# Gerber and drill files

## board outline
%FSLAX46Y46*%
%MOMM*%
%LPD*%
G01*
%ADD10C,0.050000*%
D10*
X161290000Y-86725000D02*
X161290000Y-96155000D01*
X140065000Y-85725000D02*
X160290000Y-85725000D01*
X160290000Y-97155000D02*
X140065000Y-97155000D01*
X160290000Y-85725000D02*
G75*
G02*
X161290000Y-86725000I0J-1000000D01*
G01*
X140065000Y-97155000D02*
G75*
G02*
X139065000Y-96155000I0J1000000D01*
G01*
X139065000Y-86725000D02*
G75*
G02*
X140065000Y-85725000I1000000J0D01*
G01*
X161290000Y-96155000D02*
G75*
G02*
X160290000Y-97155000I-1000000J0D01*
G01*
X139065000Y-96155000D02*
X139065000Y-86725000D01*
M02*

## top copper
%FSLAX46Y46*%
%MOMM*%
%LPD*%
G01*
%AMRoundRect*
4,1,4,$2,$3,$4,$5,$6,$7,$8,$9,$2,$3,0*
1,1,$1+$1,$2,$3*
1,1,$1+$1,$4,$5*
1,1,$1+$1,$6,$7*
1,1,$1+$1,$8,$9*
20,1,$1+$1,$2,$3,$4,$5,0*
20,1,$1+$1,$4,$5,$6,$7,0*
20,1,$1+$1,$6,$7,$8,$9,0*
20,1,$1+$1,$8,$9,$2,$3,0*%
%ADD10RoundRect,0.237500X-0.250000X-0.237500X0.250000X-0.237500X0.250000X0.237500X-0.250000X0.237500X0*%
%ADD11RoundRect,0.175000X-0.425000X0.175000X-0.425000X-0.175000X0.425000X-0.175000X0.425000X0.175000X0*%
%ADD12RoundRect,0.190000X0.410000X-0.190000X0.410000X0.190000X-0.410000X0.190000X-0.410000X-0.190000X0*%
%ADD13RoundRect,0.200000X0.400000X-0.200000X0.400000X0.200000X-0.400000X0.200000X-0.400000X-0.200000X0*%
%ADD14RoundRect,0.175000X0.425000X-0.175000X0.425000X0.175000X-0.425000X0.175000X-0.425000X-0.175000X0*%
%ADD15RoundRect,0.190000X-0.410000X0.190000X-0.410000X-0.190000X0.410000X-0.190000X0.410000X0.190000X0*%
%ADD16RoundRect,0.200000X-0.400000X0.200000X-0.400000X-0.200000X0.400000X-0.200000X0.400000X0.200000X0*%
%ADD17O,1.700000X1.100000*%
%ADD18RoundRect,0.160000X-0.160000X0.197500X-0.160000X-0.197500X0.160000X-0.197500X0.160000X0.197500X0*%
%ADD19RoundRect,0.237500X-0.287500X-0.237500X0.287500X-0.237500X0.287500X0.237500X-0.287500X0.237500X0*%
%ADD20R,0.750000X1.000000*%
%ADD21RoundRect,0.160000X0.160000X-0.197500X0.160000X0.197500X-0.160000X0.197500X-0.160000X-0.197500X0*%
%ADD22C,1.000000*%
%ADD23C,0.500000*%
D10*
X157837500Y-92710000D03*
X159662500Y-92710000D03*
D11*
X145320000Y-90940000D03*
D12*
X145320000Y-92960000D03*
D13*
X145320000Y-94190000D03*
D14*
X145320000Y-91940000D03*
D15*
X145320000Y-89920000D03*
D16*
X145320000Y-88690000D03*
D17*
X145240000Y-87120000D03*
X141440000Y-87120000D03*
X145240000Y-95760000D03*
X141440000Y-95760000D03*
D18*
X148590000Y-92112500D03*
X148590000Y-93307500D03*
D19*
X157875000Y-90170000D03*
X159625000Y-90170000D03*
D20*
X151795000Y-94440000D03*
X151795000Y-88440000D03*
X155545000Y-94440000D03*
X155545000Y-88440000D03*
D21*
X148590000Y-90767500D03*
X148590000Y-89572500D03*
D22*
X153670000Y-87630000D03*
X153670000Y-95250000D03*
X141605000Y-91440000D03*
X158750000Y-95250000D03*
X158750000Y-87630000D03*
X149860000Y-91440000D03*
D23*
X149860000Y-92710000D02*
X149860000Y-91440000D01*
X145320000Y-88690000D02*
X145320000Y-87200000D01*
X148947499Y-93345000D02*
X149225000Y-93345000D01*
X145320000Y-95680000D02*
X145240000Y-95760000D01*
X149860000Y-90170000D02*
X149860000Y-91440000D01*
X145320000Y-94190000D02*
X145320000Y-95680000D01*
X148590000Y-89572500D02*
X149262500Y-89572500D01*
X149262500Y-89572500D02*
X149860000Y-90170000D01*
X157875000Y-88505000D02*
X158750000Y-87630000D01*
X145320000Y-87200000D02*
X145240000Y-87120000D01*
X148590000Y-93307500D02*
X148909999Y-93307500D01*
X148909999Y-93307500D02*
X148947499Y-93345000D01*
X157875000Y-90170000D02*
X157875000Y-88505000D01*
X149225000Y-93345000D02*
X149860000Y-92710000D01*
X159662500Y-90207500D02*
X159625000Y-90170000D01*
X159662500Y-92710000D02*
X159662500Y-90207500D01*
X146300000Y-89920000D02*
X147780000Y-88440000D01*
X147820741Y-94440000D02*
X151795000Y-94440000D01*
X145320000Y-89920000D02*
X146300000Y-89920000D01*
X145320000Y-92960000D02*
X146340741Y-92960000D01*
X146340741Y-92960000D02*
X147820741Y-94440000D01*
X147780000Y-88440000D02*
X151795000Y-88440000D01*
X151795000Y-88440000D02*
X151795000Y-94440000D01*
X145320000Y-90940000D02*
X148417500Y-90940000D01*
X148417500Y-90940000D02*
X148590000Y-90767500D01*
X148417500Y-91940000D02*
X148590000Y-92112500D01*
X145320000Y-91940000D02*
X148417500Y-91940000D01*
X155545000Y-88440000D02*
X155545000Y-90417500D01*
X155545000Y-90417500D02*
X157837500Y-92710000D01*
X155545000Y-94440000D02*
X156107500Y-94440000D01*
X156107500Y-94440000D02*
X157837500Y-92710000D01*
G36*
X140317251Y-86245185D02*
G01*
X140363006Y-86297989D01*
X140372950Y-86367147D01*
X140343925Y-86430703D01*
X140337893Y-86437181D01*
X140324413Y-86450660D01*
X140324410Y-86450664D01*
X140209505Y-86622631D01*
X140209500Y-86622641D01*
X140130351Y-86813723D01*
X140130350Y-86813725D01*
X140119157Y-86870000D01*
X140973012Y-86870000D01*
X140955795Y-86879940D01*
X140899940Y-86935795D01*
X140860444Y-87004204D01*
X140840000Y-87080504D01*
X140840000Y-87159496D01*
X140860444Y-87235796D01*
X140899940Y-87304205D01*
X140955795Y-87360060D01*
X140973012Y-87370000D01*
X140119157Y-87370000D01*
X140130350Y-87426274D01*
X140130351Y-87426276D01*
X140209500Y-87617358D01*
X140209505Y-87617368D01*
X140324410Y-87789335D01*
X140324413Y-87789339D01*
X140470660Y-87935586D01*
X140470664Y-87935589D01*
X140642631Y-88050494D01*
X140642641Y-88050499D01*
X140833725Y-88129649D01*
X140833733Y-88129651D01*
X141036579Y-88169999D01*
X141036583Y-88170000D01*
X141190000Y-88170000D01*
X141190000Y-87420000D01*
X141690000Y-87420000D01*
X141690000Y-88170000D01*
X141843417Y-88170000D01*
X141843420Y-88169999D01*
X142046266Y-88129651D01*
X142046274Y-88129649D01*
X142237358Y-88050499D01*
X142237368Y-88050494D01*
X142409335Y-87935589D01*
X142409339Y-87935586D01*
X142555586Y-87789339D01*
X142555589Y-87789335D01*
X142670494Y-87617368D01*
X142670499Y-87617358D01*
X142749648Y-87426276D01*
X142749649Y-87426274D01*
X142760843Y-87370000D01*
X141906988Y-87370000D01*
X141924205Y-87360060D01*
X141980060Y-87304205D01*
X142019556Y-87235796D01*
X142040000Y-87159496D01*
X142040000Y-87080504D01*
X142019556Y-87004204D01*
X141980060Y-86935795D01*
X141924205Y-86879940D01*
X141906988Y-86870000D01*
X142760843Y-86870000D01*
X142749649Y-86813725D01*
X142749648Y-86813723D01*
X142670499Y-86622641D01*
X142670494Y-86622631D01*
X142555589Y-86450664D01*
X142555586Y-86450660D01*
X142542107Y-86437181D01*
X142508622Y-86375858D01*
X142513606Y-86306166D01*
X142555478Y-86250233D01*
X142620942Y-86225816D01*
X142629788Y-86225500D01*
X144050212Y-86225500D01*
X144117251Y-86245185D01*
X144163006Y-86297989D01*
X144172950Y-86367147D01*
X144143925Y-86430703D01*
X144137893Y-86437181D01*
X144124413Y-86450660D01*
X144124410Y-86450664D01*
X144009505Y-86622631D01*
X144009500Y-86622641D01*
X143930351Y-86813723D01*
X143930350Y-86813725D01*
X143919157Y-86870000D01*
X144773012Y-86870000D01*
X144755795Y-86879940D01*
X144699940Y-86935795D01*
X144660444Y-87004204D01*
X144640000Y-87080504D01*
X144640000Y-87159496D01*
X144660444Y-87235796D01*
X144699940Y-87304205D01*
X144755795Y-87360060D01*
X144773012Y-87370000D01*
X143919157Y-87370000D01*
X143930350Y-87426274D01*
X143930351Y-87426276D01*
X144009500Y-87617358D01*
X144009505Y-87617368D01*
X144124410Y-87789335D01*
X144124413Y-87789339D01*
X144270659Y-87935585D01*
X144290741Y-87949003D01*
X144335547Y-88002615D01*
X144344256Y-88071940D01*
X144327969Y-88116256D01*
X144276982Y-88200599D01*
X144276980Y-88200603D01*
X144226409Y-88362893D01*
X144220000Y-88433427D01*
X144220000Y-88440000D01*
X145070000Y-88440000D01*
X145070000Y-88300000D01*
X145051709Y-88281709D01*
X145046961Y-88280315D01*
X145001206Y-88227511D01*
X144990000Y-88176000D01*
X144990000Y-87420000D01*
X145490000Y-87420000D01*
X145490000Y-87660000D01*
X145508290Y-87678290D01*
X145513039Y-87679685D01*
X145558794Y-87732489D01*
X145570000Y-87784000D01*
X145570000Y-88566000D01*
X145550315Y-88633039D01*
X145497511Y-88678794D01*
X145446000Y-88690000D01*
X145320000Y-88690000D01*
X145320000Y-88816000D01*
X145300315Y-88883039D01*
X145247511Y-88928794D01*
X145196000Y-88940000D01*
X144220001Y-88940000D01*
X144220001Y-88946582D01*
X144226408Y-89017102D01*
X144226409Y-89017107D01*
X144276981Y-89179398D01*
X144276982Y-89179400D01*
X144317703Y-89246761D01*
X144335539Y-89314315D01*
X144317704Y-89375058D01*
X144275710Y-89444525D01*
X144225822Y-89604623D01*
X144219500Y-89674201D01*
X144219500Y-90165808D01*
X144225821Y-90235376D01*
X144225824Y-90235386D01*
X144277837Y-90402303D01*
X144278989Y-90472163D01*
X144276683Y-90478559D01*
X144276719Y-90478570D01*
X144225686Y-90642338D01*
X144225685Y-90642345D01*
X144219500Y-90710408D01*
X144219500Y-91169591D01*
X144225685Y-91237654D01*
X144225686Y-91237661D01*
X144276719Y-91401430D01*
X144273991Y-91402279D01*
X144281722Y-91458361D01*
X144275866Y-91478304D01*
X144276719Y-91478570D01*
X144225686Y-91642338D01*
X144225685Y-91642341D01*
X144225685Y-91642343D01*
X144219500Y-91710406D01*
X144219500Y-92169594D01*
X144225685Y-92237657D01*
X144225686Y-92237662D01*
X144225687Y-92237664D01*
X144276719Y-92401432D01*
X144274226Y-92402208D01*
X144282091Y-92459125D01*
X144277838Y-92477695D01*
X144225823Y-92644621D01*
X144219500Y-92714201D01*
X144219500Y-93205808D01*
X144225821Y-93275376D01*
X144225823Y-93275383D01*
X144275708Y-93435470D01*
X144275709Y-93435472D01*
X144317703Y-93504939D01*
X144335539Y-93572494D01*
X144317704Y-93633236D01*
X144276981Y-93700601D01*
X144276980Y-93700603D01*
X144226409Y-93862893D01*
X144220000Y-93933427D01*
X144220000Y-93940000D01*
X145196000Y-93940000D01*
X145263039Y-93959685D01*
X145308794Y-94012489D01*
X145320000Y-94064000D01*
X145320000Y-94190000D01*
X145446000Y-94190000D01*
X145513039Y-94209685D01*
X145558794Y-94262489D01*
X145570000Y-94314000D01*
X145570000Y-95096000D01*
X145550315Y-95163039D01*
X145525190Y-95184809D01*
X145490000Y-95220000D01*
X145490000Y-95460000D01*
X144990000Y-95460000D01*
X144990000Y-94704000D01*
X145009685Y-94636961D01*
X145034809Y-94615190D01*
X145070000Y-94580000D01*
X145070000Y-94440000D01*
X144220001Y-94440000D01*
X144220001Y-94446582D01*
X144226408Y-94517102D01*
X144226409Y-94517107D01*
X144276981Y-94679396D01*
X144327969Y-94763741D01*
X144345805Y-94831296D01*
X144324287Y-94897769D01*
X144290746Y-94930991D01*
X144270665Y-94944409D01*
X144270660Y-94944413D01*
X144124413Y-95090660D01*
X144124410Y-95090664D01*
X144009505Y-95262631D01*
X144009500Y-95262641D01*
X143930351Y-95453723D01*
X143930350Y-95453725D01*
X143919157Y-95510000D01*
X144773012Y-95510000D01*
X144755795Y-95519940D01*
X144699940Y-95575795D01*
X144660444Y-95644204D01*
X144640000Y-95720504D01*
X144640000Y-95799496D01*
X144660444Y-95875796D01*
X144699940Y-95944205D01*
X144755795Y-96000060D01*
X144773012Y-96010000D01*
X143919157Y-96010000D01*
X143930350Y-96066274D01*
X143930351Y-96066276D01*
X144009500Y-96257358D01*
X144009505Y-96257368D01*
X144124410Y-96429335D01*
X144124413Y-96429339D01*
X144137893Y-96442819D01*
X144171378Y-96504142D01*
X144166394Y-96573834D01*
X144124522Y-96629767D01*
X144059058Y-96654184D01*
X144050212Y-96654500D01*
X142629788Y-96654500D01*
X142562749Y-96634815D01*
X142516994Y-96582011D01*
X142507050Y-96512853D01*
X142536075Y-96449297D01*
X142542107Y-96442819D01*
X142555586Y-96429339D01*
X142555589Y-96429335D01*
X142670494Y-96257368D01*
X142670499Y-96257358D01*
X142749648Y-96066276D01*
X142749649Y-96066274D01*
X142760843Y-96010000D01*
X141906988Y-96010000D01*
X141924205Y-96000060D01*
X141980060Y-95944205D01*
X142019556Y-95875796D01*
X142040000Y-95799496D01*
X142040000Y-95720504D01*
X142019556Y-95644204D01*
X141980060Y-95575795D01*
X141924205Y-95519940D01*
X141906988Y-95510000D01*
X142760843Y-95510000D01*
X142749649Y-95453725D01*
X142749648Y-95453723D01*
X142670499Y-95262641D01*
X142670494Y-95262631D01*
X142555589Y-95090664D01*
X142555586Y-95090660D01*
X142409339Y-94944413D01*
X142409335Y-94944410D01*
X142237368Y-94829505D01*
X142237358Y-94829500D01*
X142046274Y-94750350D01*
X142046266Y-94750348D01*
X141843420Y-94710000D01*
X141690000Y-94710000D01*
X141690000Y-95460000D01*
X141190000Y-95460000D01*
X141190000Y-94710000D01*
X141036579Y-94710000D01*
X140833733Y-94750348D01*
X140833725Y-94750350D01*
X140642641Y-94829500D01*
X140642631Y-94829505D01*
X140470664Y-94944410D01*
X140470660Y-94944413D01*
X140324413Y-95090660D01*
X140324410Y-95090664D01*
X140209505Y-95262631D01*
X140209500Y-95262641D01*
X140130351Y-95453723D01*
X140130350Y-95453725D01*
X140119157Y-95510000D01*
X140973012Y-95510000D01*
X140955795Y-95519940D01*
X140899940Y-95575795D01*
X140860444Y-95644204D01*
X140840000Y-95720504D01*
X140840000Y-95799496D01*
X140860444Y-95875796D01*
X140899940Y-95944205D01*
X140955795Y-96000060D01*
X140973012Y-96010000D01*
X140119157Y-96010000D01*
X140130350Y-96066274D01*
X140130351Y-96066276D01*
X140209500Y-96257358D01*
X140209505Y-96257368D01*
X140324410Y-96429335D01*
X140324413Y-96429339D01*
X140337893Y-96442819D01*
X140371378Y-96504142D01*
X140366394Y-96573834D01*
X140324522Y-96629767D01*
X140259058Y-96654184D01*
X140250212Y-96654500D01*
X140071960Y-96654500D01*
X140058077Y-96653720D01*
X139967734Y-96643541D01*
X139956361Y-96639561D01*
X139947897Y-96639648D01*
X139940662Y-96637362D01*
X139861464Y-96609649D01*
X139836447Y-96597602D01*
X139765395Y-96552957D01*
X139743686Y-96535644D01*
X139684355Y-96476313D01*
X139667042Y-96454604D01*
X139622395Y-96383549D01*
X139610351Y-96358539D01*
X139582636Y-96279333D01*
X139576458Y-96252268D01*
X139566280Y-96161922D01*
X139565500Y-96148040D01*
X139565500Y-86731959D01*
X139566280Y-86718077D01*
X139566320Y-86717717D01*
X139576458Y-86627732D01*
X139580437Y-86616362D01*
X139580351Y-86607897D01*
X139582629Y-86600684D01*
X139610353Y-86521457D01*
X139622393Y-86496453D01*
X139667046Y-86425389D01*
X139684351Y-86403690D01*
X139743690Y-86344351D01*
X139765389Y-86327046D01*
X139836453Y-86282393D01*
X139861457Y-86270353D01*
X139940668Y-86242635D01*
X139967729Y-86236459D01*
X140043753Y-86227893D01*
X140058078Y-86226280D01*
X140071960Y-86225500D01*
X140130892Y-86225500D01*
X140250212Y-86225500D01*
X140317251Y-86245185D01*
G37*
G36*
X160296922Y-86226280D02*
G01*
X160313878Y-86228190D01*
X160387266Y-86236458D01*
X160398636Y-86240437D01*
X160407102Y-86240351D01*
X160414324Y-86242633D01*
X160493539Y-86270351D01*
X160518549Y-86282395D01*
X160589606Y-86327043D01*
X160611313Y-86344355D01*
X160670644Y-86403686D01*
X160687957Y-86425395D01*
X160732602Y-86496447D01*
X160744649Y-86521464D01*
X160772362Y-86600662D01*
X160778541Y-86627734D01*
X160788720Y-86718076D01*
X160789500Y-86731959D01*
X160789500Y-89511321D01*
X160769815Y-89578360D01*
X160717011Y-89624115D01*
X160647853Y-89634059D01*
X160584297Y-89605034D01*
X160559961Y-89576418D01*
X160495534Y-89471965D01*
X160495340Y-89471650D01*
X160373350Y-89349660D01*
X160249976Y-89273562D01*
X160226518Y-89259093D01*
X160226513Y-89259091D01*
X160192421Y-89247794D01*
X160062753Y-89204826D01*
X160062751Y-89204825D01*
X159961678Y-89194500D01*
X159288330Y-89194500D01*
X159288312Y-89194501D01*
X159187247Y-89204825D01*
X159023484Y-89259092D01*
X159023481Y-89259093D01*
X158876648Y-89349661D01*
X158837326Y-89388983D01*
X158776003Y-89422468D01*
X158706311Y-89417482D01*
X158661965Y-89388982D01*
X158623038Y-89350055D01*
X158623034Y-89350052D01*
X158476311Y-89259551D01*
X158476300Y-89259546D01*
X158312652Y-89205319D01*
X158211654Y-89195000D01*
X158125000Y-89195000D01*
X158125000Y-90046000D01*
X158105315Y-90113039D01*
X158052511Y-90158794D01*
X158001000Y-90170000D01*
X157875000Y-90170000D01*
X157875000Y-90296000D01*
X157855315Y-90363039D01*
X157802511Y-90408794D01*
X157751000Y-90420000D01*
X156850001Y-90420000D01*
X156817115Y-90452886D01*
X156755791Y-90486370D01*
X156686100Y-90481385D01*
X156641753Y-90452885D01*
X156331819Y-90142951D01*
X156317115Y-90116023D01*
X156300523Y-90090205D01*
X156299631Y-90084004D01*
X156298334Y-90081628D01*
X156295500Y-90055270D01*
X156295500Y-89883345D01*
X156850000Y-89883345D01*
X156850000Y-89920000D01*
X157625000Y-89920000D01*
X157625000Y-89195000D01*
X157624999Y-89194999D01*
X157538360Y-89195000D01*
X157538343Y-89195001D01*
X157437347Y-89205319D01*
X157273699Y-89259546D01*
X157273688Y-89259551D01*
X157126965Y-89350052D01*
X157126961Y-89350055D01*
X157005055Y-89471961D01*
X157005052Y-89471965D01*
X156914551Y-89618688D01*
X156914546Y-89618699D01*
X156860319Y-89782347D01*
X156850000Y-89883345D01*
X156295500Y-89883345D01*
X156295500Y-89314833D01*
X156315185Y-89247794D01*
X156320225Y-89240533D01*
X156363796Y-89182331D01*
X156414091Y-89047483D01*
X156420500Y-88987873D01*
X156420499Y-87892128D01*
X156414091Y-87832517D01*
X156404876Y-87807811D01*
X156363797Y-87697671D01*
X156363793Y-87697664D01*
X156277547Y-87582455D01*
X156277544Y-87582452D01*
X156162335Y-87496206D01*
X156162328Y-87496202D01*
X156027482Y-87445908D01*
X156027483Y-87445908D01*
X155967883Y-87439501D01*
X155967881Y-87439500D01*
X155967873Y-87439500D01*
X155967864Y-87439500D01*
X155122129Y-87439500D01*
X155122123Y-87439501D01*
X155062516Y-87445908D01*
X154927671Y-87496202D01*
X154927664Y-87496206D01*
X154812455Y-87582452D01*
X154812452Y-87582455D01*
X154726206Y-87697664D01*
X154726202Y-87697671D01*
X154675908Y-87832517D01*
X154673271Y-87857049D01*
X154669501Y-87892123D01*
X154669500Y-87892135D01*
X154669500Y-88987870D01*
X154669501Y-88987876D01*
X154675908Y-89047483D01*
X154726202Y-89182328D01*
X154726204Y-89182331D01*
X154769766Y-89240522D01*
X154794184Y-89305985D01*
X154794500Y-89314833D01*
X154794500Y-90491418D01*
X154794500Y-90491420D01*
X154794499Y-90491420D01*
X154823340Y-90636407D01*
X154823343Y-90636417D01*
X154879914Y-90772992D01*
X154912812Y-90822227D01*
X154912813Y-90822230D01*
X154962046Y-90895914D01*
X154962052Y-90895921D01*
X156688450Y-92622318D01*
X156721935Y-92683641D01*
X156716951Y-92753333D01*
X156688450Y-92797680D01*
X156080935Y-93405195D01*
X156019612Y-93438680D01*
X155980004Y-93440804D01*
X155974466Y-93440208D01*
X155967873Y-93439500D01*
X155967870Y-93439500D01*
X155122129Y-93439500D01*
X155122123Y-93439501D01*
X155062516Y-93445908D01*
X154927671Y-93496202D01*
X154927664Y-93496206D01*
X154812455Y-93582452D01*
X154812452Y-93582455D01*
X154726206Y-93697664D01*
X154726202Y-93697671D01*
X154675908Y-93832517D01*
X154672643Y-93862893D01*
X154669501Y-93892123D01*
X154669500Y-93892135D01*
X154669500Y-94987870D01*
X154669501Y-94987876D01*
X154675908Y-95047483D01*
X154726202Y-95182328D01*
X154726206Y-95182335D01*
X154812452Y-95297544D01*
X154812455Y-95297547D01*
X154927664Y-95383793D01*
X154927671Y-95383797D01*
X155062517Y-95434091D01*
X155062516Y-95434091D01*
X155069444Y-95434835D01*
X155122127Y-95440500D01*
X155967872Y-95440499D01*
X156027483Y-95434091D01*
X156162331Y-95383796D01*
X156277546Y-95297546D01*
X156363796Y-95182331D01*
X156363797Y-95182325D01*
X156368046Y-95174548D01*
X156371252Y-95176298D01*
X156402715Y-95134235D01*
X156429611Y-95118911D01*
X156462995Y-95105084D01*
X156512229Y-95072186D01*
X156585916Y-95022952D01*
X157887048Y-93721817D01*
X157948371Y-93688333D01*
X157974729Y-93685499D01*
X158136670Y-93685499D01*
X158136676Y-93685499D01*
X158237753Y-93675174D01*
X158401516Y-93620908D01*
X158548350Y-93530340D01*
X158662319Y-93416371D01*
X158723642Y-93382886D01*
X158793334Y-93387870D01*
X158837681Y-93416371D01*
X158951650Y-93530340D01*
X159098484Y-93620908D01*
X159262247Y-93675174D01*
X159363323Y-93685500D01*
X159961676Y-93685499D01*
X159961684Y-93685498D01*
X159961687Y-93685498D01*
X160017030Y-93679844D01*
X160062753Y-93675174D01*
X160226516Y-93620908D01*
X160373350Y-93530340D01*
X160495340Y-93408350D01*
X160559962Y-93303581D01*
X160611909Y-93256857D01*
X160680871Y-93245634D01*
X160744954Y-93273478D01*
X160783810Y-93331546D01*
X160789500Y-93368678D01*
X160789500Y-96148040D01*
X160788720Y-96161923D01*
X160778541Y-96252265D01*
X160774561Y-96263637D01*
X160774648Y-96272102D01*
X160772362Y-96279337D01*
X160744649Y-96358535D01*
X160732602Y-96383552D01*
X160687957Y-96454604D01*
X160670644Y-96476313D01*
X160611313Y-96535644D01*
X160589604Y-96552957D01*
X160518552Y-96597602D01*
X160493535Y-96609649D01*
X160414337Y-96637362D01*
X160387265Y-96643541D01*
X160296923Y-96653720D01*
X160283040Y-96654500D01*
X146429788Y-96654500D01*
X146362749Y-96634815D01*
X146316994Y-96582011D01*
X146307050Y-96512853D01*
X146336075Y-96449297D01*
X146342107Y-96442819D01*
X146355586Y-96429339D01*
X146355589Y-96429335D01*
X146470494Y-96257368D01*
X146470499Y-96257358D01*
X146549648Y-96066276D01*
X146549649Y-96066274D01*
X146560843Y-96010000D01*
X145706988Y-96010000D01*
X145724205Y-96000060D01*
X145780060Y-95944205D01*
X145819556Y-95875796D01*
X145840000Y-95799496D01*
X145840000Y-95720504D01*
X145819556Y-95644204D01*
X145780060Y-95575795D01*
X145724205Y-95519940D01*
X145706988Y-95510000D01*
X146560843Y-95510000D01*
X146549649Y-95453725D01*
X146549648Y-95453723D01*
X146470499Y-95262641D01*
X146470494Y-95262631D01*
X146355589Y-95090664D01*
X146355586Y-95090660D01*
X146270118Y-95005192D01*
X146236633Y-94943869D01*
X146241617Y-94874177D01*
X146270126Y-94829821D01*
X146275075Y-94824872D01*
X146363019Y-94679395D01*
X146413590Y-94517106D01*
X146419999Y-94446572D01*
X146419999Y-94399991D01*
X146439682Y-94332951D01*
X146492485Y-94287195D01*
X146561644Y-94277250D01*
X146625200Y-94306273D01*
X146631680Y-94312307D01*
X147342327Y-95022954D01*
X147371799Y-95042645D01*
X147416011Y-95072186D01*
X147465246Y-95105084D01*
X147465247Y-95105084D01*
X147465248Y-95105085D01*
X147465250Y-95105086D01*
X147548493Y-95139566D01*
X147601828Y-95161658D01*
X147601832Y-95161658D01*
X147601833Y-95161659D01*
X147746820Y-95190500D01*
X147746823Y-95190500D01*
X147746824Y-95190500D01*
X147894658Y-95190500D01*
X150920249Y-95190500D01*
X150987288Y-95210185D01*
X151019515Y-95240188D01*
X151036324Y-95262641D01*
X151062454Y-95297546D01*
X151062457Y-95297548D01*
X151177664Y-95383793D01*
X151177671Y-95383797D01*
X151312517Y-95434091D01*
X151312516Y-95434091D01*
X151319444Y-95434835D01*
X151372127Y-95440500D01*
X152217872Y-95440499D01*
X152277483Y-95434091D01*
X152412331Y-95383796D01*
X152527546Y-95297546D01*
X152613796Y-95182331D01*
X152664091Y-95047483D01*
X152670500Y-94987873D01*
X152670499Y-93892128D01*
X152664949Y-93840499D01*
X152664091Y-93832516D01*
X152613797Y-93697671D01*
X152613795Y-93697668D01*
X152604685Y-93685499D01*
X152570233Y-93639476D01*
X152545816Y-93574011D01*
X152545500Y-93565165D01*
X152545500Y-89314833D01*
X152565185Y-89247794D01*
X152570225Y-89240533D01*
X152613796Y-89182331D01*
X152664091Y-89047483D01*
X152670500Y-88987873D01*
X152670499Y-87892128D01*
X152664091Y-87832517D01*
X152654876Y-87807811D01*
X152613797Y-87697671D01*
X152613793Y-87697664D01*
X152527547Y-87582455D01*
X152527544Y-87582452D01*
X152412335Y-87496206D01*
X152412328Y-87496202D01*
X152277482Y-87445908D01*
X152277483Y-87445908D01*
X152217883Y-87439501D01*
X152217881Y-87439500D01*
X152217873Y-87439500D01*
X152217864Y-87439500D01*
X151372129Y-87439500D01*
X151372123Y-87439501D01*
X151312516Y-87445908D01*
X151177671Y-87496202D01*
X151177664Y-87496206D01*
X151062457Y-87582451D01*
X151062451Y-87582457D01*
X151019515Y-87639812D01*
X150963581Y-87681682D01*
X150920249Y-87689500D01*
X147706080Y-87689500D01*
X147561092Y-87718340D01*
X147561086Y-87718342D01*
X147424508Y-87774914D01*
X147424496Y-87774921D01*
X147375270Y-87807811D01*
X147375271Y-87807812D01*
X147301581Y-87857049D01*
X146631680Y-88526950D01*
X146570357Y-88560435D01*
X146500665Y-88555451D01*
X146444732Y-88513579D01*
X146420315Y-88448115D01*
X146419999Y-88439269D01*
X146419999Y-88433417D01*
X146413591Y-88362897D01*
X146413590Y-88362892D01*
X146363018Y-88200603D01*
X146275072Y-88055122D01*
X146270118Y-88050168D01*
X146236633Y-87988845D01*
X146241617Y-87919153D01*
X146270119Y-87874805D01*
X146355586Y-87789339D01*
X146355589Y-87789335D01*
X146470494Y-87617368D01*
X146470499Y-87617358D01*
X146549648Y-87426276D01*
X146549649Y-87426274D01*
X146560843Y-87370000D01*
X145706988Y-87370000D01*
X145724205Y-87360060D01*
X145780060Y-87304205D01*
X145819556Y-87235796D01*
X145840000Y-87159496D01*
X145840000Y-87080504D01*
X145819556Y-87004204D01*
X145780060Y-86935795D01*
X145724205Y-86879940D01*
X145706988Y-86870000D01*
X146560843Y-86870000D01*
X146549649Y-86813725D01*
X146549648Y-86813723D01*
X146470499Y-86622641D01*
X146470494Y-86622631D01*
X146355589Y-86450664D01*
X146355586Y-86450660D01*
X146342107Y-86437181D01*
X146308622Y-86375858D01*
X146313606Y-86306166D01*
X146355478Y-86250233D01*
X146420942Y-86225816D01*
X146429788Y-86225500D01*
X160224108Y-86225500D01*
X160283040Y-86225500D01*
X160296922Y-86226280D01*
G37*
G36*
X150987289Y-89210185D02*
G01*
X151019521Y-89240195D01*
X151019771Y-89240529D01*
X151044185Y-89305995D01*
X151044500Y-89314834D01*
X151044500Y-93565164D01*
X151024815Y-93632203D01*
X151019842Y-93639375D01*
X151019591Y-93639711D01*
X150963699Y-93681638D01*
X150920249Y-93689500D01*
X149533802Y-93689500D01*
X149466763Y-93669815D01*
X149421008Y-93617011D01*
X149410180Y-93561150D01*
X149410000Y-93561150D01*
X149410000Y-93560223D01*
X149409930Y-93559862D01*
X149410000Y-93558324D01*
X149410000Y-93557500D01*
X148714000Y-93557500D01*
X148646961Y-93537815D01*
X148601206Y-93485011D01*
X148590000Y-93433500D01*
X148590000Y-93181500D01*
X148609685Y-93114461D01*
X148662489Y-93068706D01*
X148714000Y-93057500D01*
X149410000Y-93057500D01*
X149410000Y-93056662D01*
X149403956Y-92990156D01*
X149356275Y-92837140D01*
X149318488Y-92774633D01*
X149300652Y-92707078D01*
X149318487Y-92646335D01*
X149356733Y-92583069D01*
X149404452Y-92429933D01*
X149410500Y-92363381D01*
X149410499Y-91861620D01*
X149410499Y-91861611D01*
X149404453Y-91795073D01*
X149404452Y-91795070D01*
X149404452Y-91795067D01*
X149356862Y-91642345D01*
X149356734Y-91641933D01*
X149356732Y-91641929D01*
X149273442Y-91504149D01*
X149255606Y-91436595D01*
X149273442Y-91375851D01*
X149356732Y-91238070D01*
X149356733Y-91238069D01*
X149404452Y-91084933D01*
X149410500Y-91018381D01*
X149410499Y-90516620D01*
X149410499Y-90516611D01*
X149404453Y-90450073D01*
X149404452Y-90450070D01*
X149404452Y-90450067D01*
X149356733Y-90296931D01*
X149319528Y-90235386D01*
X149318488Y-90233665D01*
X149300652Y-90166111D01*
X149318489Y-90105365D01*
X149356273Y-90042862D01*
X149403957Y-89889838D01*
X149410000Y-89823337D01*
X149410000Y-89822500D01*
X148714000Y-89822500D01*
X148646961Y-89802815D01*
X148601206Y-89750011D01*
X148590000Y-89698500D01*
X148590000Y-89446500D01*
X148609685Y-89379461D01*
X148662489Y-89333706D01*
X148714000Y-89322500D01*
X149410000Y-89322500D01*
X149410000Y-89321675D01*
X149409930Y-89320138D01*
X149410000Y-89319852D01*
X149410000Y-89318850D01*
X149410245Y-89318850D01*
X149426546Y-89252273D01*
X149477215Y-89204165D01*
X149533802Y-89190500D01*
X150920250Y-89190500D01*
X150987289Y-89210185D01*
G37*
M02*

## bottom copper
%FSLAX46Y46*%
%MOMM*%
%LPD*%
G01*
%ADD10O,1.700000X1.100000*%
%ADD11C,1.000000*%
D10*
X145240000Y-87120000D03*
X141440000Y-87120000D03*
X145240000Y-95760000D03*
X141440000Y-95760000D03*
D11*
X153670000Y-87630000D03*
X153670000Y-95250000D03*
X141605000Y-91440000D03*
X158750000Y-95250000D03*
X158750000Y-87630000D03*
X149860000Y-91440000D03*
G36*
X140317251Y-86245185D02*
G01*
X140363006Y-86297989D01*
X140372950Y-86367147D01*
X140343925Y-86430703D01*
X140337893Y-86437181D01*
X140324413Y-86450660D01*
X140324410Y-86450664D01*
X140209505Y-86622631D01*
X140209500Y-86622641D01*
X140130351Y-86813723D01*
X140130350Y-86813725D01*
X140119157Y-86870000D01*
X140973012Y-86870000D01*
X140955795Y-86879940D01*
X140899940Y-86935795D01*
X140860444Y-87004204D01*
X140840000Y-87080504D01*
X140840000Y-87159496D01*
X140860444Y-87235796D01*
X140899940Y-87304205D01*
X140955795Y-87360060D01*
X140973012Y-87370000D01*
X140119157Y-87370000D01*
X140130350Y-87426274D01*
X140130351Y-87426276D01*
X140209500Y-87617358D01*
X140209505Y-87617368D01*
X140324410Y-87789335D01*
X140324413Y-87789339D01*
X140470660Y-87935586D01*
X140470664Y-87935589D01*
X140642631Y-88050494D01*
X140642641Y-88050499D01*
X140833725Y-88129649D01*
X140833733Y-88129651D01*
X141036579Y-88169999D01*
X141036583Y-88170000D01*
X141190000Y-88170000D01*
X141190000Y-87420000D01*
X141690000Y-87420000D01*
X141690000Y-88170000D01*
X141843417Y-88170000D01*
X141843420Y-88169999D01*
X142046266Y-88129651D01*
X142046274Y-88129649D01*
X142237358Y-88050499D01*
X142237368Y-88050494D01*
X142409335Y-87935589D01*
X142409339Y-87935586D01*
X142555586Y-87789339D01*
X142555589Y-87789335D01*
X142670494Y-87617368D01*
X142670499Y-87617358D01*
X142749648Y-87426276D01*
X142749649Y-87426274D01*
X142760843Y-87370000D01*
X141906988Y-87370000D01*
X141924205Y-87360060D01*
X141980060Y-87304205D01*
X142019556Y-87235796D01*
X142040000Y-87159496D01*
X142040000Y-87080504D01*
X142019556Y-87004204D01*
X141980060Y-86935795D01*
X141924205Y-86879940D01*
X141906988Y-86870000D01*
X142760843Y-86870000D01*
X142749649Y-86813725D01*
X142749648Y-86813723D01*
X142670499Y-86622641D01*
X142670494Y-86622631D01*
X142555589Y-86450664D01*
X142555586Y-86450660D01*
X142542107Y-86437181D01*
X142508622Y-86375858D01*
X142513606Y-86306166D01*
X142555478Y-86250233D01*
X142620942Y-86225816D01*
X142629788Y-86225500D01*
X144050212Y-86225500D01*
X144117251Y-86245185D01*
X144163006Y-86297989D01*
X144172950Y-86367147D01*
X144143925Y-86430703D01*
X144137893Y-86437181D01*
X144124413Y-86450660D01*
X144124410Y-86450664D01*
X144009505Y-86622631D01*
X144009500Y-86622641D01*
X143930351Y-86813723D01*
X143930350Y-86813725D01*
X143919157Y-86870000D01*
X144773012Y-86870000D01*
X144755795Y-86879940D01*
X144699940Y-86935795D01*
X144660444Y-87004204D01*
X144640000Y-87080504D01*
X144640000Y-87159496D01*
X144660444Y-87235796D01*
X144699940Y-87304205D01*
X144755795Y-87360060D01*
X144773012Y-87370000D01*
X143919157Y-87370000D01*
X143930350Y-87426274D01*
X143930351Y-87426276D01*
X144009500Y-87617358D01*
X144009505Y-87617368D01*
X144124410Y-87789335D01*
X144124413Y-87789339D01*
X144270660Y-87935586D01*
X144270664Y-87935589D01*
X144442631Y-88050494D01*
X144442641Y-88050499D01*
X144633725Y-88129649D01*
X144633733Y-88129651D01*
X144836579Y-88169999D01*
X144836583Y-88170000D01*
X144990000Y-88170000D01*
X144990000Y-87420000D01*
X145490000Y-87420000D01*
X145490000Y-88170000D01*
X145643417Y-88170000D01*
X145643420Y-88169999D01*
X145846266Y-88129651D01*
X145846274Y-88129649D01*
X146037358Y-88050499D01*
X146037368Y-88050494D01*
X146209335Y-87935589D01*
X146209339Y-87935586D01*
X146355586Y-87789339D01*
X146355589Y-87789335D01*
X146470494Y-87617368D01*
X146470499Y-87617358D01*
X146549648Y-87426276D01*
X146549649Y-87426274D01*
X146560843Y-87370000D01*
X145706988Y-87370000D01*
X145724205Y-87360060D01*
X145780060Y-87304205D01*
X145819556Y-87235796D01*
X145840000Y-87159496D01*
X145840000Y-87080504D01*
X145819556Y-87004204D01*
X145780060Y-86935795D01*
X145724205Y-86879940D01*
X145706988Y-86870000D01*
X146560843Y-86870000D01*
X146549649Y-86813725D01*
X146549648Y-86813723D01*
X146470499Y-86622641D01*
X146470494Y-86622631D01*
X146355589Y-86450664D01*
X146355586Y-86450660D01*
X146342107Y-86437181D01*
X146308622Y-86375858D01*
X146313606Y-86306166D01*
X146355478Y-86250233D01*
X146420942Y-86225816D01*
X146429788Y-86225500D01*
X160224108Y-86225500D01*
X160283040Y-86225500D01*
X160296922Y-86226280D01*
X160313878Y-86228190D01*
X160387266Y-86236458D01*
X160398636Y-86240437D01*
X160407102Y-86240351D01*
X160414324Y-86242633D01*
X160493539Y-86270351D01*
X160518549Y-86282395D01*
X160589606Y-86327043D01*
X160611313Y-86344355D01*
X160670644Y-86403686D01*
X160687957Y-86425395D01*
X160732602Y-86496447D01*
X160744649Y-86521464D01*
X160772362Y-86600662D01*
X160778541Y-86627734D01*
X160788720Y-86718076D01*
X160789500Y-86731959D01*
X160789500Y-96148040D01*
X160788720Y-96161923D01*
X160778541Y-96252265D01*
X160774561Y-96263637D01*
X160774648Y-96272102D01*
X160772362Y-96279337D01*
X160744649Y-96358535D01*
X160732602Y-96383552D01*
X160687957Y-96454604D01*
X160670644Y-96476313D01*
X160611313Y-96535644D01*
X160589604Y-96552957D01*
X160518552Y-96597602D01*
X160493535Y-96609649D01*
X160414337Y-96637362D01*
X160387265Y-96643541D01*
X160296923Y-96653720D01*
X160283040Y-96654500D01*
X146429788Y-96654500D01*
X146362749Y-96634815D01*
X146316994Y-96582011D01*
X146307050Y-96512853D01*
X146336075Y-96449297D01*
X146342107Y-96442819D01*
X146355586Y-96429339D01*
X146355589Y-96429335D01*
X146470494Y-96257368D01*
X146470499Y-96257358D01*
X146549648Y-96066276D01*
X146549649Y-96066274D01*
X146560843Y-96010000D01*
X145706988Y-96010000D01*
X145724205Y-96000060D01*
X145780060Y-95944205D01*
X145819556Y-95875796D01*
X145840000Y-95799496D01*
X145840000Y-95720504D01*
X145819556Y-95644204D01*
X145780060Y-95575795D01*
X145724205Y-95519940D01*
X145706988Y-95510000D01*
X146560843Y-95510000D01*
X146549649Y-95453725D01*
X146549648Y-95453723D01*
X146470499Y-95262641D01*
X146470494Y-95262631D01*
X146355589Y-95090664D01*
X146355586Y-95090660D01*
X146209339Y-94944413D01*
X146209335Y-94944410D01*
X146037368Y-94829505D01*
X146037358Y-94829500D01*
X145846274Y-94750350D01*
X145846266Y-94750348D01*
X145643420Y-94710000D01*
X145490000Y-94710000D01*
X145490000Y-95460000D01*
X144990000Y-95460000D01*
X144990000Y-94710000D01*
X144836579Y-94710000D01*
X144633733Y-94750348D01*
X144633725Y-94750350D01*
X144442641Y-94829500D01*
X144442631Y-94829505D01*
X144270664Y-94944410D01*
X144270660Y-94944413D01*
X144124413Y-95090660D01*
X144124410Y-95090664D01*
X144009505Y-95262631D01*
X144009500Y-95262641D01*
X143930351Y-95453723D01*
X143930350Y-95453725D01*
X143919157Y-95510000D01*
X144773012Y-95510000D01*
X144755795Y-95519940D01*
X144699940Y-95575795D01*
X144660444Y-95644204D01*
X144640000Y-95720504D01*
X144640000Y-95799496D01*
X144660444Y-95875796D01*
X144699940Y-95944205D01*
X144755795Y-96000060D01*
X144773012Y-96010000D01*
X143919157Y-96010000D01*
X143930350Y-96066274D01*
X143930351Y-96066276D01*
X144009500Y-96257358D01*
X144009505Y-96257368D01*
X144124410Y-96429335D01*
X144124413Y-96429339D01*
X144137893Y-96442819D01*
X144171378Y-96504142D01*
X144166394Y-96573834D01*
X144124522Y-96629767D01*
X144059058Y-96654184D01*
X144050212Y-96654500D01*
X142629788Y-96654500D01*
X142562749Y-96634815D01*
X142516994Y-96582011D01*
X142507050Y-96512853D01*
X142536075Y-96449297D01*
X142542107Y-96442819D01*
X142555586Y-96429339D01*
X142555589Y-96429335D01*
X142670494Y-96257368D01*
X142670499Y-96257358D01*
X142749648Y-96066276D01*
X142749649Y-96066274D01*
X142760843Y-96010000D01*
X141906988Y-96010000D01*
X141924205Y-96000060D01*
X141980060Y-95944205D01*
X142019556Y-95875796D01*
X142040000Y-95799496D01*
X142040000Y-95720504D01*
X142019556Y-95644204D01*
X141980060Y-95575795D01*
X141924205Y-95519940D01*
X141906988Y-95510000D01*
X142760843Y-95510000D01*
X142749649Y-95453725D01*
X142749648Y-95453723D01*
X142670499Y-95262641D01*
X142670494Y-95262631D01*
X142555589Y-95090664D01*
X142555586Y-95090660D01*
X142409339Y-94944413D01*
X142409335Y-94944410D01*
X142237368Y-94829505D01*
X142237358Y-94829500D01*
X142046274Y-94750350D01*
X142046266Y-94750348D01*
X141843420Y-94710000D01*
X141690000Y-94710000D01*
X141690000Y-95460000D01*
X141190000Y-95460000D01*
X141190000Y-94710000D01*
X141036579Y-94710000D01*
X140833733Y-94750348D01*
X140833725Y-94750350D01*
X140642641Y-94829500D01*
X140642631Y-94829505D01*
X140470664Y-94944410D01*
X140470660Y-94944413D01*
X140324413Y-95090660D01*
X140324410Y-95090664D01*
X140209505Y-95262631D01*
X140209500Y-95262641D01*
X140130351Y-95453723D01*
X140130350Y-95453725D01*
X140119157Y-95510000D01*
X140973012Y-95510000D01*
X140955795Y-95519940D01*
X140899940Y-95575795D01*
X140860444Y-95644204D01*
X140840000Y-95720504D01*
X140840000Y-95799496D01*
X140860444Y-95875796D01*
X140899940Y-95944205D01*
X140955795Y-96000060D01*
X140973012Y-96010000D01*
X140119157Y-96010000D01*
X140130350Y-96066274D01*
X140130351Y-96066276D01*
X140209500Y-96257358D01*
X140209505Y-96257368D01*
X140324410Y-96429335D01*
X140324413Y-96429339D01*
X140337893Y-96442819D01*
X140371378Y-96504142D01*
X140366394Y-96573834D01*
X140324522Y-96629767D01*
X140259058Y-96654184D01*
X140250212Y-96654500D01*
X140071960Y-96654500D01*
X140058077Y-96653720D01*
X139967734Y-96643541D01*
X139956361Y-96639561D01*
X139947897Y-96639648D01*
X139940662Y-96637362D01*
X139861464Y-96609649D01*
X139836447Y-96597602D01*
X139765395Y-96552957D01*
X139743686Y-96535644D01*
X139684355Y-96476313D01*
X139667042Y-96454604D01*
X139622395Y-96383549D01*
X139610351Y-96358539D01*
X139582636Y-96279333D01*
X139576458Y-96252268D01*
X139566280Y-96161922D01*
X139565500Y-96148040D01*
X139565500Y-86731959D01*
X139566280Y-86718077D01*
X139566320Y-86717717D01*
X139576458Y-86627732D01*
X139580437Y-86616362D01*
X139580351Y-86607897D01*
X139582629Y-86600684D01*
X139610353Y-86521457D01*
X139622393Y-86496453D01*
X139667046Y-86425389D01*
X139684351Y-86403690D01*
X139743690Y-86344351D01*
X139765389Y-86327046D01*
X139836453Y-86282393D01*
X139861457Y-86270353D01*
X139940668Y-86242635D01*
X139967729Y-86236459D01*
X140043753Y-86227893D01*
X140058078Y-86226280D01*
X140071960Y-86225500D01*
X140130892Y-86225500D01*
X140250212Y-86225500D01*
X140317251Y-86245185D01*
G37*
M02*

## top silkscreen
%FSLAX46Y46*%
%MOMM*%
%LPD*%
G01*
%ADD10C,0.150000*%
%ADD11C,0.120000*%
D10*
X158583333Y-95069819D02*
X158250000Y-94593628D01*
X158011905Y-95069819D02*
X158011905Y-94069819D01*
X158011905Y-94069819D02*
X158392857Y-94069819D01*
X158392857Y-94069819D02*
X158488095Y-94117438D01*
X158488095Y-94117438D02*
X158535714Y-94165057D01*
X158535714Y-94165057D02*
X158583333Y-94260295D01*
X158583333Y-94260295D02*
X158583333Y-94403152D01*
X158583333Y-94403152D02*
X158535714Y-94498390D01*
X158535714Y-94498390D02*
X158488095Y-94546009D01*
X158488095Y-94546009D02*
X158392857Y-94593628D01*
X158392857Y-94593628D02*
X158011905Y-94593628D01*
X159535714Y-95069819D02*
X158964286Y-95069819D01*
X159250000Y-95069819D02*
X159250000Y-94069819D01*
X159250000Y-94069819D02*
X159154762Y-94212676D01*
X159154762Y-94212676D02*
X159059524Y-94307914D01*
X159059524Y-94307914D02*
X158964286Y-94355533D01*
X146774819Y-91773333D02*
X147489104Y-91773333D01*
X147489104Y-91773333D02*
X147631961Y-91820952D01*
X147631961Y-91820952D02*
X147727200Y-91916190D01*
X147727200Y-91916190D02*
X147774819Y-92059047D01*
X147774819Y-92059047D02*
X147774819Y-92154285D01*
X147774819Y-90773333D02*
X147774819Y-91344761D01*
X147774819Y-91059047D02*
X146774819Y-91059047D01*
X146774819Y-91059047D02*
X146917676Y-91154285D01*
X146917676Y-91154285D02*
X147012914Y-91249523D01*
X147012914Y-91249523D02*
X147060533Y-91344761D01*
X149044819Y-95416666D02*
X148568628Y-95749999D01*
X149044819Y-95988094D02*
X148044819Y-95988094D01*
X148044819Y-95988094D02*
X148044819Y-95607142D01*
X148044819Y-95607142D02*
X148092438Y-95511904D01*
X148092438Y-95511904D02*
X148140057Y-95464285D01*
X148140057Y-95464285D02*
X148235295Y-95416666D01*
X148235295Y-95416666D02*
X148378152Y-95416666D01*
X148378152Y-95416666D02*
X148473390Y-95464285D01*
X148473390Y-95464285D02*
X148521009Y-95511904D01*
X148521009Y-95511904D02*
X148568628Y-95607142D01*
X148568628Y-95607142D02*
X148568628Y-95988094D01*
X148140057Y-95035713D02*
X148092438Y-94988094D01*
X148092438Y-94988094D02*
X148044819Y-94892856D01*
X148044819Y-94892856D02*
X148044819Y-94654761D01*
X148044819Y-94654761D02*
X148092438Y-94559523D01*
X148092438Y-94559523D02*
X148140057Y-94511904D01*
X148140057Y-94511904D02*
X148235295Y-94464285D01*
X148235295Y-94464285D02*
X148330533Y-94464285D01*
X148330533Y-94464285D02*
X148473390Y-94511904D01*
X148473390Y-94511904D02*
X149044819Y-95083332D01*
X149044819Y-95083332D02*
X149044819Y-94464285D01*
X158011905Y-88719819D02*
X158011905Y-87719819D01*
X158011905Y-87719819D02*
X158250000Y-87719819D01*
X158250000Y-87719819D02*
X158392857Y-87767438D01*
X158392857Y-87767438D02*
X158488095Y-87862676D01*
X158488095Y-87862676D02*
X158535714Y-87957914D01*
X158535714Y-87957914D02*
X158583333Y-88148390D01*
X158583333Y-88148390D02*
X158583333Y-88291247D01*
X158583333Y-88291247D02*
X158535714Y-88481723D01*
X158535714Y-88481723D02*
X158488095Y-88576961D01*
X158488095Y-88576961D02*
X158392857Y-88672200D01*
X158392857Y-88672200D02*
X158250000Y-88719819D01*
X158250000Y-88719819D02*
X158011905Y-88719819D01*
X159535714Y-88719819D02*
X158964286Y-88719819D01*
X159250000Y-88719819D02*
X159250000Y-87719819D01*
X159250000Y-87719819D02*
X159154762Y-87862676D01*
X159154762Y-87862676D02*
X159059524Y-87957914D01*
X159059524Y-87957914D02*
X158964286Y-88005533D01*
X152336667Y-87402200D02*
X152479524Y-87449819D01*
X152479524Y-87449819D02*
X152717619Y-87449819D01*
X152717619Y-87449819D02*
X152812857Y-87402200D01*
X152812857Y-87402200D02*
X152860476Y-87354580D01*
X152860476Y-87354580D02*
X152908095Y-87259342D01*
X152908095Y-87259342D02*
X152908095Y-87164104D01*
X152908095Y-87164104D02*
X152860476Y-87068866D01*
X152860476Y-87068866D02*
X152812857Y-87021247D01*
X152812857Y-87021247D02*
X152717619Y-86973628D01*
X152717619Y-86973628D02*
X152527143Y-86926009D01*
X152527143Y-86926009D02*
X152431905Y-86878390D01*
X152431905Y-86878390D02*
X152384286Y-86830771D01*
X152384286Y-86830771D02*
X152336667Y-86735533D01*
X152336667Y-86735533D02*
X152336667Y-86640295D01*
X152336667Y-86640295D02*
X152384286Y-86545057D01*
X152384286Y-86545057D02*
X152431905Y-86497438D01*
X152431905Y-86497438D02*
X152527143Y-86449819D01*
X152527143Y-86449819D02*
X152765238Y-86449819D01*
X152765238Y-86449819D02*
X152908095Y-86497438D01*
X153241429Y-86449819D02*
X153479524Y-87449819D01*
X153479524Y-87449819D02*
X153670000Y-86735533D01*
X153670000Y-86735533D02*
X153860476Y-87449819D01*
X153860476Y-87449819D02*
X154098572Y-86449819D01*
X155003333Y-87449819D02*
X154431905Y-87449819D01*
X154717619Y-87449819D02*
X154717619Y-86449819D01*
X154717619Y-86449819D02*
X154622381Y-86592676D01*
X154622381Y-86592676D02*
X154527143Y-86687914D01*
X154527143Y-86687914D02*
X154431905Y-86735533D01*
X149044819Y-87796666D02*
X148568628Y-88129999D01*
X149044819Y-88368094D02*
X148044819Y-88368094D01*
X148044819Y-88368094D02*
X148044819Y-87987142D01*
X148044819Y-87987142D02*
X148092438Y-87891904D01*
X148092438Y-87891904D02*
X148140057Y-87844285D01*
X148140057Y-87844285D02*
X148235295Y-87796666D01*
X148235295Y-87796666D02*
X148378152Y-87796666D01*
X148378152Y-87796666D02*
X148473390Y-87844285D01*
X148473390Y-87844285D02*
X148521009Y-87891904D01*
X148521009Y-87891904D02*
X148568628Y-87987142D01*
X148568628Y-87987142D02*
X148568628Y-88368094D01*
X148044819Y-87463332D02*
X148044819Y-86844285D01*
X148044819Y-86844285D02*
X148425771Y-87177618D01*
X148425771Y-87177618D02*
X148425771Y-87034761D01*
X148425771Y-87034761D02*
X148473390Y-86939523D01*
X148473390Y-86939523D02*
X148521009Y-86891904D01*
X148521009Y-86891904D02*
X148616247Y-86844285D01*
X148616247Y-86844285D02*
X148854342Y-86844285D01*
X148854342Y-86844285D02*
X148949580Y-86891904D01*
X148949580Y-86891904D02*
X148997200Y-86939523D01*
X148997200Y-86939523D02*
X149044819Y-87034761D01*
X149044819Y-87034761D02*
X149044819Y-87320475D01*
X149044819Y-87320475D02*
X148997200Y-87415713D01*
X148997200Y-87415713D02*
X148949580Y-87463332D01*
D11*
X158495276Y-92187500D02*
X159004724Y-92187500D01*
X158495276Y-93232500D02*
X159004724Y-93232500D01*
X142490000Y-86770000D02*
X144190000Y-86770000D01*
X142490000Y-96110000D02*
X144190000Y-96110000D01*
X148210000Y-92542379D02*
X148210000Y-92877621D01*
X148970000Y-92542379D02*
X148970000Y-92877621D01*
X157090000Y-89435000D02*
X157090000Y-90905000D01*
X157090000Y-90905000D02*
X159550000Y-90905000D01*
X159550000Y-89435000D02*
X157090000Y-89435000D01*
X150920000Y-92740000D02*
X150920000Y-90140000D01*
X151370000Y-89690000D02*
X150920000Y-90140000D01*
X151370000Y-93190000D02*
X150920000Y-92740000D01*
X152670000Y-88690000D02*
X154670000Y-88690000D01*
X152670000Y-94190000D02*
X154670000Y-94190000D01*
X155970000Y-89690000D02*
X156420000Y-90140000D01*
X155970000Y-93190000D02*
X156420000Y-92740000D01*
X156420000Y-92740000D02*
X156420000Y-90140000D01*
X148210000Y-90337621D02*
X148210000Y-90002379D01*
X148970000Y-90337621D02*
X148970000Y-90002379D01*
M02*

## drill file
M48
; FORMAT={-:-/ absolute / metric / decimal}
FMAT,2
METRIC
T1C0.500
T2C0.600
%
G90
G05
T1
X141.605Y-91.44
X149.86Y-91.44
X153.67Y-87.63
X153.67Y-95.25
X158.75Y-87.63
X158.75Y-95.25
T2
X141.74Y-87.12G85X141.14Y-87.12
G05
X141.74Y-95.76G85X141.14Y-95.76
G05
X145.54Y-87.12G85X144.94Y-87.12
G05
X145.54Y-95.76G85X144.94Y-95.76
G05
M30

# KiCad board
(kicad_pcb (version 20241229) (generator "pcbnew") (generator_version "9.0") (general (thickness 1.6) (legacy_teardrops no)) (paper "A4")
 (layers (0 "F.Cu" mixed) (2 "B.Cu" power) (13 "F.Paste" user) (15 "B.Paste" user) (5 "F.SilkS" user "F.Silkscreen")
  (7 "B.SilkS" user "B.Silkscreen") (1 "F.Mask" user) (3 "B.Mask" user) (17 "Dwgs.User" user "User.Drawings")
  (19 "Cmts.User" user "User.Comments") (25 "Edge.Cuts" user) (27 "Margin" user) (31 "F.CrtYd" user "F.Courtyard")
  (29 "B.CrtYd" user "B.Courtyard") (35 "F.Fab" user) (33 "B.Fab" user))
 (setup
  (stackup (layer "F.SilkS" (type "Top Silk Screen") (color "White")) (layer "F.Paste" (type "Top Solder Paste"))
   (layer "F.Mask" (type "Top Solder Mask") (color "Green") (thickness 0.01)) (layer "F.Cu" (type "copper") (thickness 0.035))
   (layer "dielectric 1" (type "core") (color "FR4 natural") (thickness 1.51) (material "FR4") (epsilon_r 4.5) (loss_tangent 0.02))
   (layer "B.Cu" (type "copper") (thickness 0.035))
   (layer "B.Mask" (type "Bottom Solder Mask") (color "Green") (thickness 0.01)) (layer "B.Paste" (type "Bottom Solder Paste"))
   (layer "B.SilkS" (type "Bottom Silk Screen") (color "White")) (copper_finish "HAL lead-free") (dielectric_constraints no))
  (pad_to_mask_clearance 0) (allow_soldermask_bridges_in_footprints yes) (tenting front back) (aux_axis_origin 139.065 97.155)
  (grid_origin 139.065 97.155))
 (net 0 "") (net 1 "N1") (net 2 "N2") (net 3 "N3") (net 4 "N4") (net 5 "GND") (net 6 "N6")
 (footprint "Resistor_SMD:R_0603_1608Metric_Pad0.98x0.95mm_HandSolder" (layer "F.Cu") (at 158.75 92.71)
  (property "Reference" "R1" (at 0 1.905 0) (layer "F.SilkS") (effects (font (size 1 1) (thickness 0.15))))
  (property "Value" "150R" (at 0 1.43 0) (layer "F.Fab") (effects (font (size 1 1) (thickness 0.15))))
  (fp_line (start -0.254724 -0.5225) (end 0.254724 -0.5225) (stroke (width 0.12) (type solid)) (layer "F.SilkS"))
  (fp_line (start -0.254724 0.5225) (end 0.254724 0.5225) (stroke (width 0.12) (type solid)) (layer "F.SilkS"))
  (pad "1" smd roundrect (at -0.9125 0) (size 0.975 0.95) (layers "F.Cu" "F.Mask" "F.Paste") (roundrect_rratio 0.25) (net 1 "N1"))
  (pad "2" smd roundrect (at 0.9125 0) (size 0.975 0.95) (layers "F.Cu" "F.Mask" "F.Paste") (roundrect_rratio 0.25) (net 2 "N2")))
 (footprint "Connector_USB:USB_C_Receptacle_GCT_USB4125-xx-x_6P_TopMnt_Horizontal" (layer "F.Cu") (at 142.24 91.44 -90)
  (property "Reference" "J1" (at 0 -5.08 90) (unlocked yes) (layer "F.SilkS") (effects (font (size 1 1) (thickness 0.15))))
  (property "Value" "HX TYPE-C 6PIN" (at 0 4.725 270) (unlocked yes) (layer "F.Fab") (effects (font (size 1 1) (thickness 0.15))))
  (fp_line (start -4.67 -0.25) (end -4.67 -1.95) (stroke (width 0.12) (type solid)) (layer "F.SilkS"))
  (fp_line (start 4.67 -0.25) (end 4.67 -1.95) (stroke (width 0.12) (type solid)) (layer "F.SilkS"))
  (pad "A5" smd roundrect (at -0.5 -3.08 270) (size 0.7 1.2) (layers "F.Cu" "F.Mask" "F.Paste") (roundrect_rratio 0.25) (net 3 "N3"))
  (pad "A9" smd roundrect (at 1.52 -3.08 90) (size 0.76 1.2) (layers "F.Cu" "F.Mask" "F.Paste") (roundrect_rratio 0.25) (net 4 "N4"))
  (pad "A12" smd roundrect (at 2.75 -3.08 90) (size 0.8 1.2) (layers "F.Cu" "F.Mask" "F.Paste") (roundrect_rratio 0.25) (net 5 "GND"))
  (pad "B5" smd roundrect (at 0.5 -3.08 90) (size 0.7 1.2) (layers "F.Cu" "F.Mask" "F.Paste") (roundrect_rratio 0.25) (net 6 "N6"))
  (pad "B9" smd roundrect (at -1.52 -3.08 270) (size 0.76 1.2) (layers "F.Cu" "F.Mask" "F.Paste") (roundrect_rratio 0.25) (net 4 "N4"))
  (pad "B12" smd roundrect (at -2.75 -3.08 270) (size 0.8 1.2) (layers "F.Cu" "F.Mask" "F.Paste") (roundrect_rratio 0.25) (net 5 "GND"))
  (pad "S1" thru_hole oval (at -4.32 -3 270) (size 1.1 1.7) (drill oval 0.6 1.2) (layers "*.Cu" "*.Mask" "F.Paste")
   (remove_unused_layers no) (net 5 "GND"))
  (pad "S1" thru_hole oval (at -4.32 0.8 270) (size 1.1 1.7) (drill oval 0.6 1.2) (layers "*.Cu" "*.Mask" "F.Paste")
   (remove_unused_layers no) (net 5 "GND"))
  (pad "S1" thru_hole oval (at 4.32 -3 270) (size 1.1 1.7) (drill oval 0.6 1.2) (layers "*.Cu" "*.Mask" "F.Paste") (remove_unused_layers no)
   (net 5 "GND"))
  (pad "S1" thru_hole oval (at 4.32 0.8 270) (size 1.1 1.7) (drill oval 0.6 1.2) (layers "*.Cu" "*.Mask" "F.Paste")
   (remove_unused_layers no) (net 5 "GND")))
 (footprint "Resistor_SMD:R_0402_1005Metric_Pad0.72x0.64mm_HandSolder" (layer "F.Cu") (at 148.59 92.71 -90)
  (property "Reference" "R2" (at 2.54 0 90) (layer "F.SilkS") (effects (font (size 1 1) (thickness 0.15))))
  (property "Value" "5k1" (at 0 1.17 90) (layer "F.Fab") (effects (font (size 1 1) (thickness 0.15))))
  (fp_line (start -0.167621 0.38) (end 0.167621 0.38) (stroke (width 0.12) (type solid)) (layer "F.SilkS"))
  (fp_line (start -0.167621 -0.38) (end 0.167621 -0.38) (stroke (width 0.12) (type solid)) (layer "F.SilkS"))
  (pad "1" smd roundrect (at -0.5975 0 270) (size 0.715 0.64) (layers "F.Cu" "F.Mask" "F.Paste") (roundrect_rratio 0.25) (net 6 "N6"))
  (pad "2" smd roundrect (at 0.5975 0 270) (size 0.715 0.64) (layers "F.Cu" "F.Mask" "F.Paste") (roundrect_rratio 0.25) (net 5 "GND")))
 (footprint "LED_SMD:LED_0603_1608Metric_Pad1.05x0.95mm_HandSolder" (layer "F.Cu") (at 158.75 90.17)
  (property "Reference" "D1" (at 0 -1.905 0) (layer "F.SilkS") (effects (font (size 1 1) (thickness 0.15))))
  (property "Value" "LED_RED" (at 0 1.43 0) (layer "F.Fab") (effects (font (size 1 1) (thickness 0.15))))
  (fp_line (start -1.66 -0.735) (end -1.66 0.735) (stroke (width 0.12) (type solid)) (layer "F.SilkS"))
  (fp_line (start -1.66 0.735) (end 0.8 0.735) (stroke (width 0.12) (type solid)) (layer "F.SilkS"))
  (fp_line (start 0.8 -0.735) (end -1.66 -0.735) (stroke (width 0.12) (type solid)) (layer "F.SilkS"))
  (pad "1" smd roundrect (at -0.875 0) (size 1.05 0.95) (layers "F.Cu" "F.Mask" "F.Paste") (roundrect_rratio 0.25) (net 5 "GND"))
  (pad "2" smd roundrect (at 0.875 0) (size 1.05 0.95) (layers "F.Cu" "F.Mask" "F.Paste") (roundrect_rratio 0.25) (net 2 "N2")))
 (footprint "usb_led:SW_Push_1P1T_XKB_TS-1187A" (layer "F.Cu") (at 153.67 91.44 90)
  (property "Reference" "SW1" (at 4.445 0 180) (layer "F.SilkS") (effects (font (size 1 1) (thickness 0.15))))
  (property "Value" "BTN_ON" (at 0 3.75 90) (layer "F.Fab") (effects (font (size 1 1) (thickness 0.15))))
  (fp_line (start -1.3 -2.75) (end 1.3 -2.75) (stroke (width 0.12) (type solid)) (layer "F.SilkS"))
  (fp_line (start 1.75 -2.3) (end 1.3 -2.75) (stroke (width 0.12) (type solid)) (layer "F.SilkS"))
  (fp_line (start -1.75 -2.3) (end -1.3 -2.75) (stroke (width 0.12) (type solid)) (layer "F.SilkS"))
  (fp_line (start 2.75 -1) (end 2.75 1) (stroke (width 0.12) (type solid)) (layer "F.SilkS"))
  (fp_line (start -2.75 -1) (end -2.75 1) (stroke (width 0.12) (type solid)) (layer "F.SilkS"))
  (fp_line (start 1.75 2.3) (end 1.3 2.75) (stroke (width 0.12) (type solid)) (layer "F.SilkS"))
  (fp_line (start -1.75 2.3) (end -1.3 2.75) (stroke (width 0.12) (type solid)) (layer "F.SilkS"))
  (fp_line (start -1.3 2.75) (end 1.3 2.75) (stroke (width 0.12) (type solid)) (layer "F.SilkS"))
  (pad "1" smd rect (at -3 -1.875 90) (size 1 0.75) (layers "F.Cu" "F.Mask" "F.Paste") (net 4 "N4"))
  (pad "1" smd rect (at 3 -1.875 90) (size 1 0.75) (layers "F.Cu" "F.Mask" "F.Paste") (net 4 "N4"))
  (pad "2" smd rect (at -3 1.875 90) (size 1 0.75) (layers "F.Cu" "F.Mask" "F.Paste") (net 1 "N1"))
  (pad "2" smd rect (at 3 1.875 90) (size 1 0.75) (layers "F.Cu" "F.Mask" "F.Paste") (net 1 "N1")))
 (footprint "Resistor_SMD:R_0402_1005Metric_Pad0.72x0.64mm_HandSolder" (layer "F.Cu") (at 148.59 90.17 90)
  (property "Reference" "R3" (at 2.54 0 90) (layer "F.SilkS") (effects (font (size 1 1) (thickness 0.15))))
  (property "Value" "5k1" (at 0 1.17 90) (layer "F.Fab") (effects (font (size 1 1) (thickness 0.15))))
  (fp_line (start -0.167621 -0.38) (end 0.167621 -0.38) (stroke (width 0.12) (type solid)) (layer "F.SilkS"))
  (fp_line (start -0.167621 0.38) (end 0.167621 0.38) (stroke (width 0.12) (type solid)) (layer "F.SilkS"))
  (pad "1" smd roundrect (at -0.5975 0 90) (size 0.715 0.64) (layers "F.Cu" "F.Mask" "F.Paste") (roundrect_rratio 0.25) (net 3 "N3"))
  (pad "2" smd roundrect (at 0.5975 0 90) (size 0.715 0.64) (layers "F.Cu" "F.Mask" "F.Paste") (roundrect_rratio 0.25) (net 5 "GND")))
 (gr_line (start 161.29 86.725) (end 161.29 96.155) (stroke (width 0.05) (type default)) (layer "Edge.Cuts"))
 (gr_line (start 140.065 85.725) (end 160.29 85.725) (stroke (width 0.05) (type default)) (layer "Edge.Cuts"))
 (gr_line (start 160.29 97.155) (end 140.065 97.155) (stroke (width 0.05) (type default)) (layer "Edge.Cuts"))
 (gr_arc (start 160.29 85.725) (mid 160.997107 86.017893) (end 161.29 86.725) (stroke (width 0.05) (type default)) (layer "Edge.Cuts"))
 (gr_arc (start 140.065 97.155) (mid 139.357893 96.862107) (end 139.065 96.155) (stroke (width 0.05) (type default)) (layer "Edge.Cuts"))
 (gr_arc (start 139.065 86.725) (mid 139.357893 86.017893) (end 140.065 85.725) (stroke (width 0.05) (type default)) (layer "Edge.Cuts"))
 (gr_arc (start 161.29 96.155) (mid 160.997107 96.862107) (end 160.29 97.155) (stroke (width 0.05) (type default)) (layer "Edge.Cuts"))
 (gr_line (start 139.065 96.155) (end 139.065 86.725) (stroke (width 0.05) (type default)) (layer "Edge.Cuts"))
 (segment (start 149.86 92.71) (end 149.86 91.44) (width 0.5) (layer "F.Cu") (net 5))
 (segment (start 145.32 88.69) (end 145.32 87.2) (width 0.5) (layer "F.Cu") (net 5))
 (segment (start 148.947499 93.345) (end 149.225 93.345) (width 0.5) (layer "F.Cu") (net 5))
 (segment (start 145.32 95.68) (end 145.24 95.76) (width 0.5) (layer "F.Cu") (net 5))
 (segment (start 149.86 90.17) (end 149.86 91.44) (width 0.5) (layer "F.Cu") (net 5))
 (segment (start 145.32 94.19) (end 145.32 95.68) (width 0.5) (layer "F.Cu") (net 5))
 (segment (start 148.59 89.5725) (end 149.2625 89.5725) (width 0.5) (layer "F.Cu") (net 5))
 (segment (start 149.2625 89.5725) (end 149.86 90.17) (width 0.5) (layer "F.Cu") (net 5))
 (segment (start 157.875 88.505) (end 158.75 87.63) (width 0.5) (layer "F.Cu") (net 5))
 (segment (start 145.32 87.2) (end 145.24 87.12) (width 0.5) (layer "F.Cu") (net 5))
 (segment (start 148.59 93.3075) (end 148.909999 93.3075) (width 0.5) (layer "F.Cu") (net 5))
 (segment (start 148.909999 93.3075) (end 148.947499 93.345) (width 0.5) (layer "F.Cu") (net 5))
 (segment (start 157.875 90.17) (end 157.875 88.505) (width 0.5) (layer "F.Cu") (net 5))
 (segment (start 149.225 93.345) (end 149.86 92.71) (width 0.5) (layer "F.Cu") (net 5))
 (via (at 153.67 87.63) (size 1) (drill 0.5) (layers "F.Cu" "B.Cu") (free yes) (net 5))
 (via (at 153.67 95.25) (size 1) (drill 0.5) (layers "F.Cu" "B.Cu") (free yes) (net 5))
 (via (at 141.605 91.44) (size 1) (drill 0.5) (layers "F.Cu" "B.Cu") (free yes) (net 5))
 (via (at 158.75 95.25) (size 1) (drill 0.5) (layers "F.Cu" "B.Cu") (free yes) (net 5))
 (via (at 158.75 87.63) (size 1) (drill 0.5) (layers "F.Cu" "B.Cu") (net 5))
 (via (at 149.86 91.44) (size 1) (drill 0.5) (layers "F.Cu" "B.Cu") (free yes) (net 5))
 (segment (start 159.6625 90.2075) (end 159.625 90.17) (width 0.5) (layer "F.Cu") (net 2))
 (segment (start 159.6625 92.71) (end 159.6625 90.2075) (width 0.5) (layer "F.Cu") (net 2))
 (segment (start 146.3 89.92) (end 147.78 88.44) (width 0.5) (layer "F.Cu") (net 4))
 (segment (start 147.820741 94.44) (end 151.795 94.44) (width 0.5) (layer "F.Cu") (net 4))
 (segment (start 145.32 89.92) (end 146.3 89.92) (width 0.5) (layer "F.Cu") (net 4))
 (segment (start 145.32 92.96) (end 146.340741 92.96) (width 0.5) (layer "F.Cu") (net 4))
 (segment (start 146.340741 92.96) (end 147.820741 94.44) (width 0.5) (layer "F.Cu") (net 4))
 (segment (start 147.78 88.44) (end 151.795 88.44) (width 0.5) (layer "F.Cu") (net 4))
 (segment (start 151.795 88.44) (end 151.795 94.44) (width 0.5) (layer "F.Cu") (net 4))
 (segment (start 145.32 90.94) (end 148.4175 90.94) (width 0.5) (layer "F.Cu") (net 3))
 (segment (start 148.4175 90.94) (end 148.59 90.7675) (width 0.5) (layer "F.Cu") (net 3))
 (segment (start 148.4175 91.94) (end 148.59 92.1125) (width 0.5) (layer "F.Cu") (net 6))
 (segment (start 145.32 91.94) (end 148.4175 91.94) (width 0.5) (layer "F.Cu") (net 6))
 (segment (start 155.545 88.44) (end 155.545 90.4175) (width 0.5) (layer "F.Cu") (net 1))
 (segment (start 155.545 90.4175) (end 157.8375 92.71) (width 0.5) (layer "F.Cu") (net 1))
 (segment (start 155.545 94.44) (end 156.1075 94.44) (width 0.5) (layer "F.Cu") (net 1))
 (segment (start 156.1075 94.44) (end 157.8375 92.71) (width 0.5) (layer "F.Cu") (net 1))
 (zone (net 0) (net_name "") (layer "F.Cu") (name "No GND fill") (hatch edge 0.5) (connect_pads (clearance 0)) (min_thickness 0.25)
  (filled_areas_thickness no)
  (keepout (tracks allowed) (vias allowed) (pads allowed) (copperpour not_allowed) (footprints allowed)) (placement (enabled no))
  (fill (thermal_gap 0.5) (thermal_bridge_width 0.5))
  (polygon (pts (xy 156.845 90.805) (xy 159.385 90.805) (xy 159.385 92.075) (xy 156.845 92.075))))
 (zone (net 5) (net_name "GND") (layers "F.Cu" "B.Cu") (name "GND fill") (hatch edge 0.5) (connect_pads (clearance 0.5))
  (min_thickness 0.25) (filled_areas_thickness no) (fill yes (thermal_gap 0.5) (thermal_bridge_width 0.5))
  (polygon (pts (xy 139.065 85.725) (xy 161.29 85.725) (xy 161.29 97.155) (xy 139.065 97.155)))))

